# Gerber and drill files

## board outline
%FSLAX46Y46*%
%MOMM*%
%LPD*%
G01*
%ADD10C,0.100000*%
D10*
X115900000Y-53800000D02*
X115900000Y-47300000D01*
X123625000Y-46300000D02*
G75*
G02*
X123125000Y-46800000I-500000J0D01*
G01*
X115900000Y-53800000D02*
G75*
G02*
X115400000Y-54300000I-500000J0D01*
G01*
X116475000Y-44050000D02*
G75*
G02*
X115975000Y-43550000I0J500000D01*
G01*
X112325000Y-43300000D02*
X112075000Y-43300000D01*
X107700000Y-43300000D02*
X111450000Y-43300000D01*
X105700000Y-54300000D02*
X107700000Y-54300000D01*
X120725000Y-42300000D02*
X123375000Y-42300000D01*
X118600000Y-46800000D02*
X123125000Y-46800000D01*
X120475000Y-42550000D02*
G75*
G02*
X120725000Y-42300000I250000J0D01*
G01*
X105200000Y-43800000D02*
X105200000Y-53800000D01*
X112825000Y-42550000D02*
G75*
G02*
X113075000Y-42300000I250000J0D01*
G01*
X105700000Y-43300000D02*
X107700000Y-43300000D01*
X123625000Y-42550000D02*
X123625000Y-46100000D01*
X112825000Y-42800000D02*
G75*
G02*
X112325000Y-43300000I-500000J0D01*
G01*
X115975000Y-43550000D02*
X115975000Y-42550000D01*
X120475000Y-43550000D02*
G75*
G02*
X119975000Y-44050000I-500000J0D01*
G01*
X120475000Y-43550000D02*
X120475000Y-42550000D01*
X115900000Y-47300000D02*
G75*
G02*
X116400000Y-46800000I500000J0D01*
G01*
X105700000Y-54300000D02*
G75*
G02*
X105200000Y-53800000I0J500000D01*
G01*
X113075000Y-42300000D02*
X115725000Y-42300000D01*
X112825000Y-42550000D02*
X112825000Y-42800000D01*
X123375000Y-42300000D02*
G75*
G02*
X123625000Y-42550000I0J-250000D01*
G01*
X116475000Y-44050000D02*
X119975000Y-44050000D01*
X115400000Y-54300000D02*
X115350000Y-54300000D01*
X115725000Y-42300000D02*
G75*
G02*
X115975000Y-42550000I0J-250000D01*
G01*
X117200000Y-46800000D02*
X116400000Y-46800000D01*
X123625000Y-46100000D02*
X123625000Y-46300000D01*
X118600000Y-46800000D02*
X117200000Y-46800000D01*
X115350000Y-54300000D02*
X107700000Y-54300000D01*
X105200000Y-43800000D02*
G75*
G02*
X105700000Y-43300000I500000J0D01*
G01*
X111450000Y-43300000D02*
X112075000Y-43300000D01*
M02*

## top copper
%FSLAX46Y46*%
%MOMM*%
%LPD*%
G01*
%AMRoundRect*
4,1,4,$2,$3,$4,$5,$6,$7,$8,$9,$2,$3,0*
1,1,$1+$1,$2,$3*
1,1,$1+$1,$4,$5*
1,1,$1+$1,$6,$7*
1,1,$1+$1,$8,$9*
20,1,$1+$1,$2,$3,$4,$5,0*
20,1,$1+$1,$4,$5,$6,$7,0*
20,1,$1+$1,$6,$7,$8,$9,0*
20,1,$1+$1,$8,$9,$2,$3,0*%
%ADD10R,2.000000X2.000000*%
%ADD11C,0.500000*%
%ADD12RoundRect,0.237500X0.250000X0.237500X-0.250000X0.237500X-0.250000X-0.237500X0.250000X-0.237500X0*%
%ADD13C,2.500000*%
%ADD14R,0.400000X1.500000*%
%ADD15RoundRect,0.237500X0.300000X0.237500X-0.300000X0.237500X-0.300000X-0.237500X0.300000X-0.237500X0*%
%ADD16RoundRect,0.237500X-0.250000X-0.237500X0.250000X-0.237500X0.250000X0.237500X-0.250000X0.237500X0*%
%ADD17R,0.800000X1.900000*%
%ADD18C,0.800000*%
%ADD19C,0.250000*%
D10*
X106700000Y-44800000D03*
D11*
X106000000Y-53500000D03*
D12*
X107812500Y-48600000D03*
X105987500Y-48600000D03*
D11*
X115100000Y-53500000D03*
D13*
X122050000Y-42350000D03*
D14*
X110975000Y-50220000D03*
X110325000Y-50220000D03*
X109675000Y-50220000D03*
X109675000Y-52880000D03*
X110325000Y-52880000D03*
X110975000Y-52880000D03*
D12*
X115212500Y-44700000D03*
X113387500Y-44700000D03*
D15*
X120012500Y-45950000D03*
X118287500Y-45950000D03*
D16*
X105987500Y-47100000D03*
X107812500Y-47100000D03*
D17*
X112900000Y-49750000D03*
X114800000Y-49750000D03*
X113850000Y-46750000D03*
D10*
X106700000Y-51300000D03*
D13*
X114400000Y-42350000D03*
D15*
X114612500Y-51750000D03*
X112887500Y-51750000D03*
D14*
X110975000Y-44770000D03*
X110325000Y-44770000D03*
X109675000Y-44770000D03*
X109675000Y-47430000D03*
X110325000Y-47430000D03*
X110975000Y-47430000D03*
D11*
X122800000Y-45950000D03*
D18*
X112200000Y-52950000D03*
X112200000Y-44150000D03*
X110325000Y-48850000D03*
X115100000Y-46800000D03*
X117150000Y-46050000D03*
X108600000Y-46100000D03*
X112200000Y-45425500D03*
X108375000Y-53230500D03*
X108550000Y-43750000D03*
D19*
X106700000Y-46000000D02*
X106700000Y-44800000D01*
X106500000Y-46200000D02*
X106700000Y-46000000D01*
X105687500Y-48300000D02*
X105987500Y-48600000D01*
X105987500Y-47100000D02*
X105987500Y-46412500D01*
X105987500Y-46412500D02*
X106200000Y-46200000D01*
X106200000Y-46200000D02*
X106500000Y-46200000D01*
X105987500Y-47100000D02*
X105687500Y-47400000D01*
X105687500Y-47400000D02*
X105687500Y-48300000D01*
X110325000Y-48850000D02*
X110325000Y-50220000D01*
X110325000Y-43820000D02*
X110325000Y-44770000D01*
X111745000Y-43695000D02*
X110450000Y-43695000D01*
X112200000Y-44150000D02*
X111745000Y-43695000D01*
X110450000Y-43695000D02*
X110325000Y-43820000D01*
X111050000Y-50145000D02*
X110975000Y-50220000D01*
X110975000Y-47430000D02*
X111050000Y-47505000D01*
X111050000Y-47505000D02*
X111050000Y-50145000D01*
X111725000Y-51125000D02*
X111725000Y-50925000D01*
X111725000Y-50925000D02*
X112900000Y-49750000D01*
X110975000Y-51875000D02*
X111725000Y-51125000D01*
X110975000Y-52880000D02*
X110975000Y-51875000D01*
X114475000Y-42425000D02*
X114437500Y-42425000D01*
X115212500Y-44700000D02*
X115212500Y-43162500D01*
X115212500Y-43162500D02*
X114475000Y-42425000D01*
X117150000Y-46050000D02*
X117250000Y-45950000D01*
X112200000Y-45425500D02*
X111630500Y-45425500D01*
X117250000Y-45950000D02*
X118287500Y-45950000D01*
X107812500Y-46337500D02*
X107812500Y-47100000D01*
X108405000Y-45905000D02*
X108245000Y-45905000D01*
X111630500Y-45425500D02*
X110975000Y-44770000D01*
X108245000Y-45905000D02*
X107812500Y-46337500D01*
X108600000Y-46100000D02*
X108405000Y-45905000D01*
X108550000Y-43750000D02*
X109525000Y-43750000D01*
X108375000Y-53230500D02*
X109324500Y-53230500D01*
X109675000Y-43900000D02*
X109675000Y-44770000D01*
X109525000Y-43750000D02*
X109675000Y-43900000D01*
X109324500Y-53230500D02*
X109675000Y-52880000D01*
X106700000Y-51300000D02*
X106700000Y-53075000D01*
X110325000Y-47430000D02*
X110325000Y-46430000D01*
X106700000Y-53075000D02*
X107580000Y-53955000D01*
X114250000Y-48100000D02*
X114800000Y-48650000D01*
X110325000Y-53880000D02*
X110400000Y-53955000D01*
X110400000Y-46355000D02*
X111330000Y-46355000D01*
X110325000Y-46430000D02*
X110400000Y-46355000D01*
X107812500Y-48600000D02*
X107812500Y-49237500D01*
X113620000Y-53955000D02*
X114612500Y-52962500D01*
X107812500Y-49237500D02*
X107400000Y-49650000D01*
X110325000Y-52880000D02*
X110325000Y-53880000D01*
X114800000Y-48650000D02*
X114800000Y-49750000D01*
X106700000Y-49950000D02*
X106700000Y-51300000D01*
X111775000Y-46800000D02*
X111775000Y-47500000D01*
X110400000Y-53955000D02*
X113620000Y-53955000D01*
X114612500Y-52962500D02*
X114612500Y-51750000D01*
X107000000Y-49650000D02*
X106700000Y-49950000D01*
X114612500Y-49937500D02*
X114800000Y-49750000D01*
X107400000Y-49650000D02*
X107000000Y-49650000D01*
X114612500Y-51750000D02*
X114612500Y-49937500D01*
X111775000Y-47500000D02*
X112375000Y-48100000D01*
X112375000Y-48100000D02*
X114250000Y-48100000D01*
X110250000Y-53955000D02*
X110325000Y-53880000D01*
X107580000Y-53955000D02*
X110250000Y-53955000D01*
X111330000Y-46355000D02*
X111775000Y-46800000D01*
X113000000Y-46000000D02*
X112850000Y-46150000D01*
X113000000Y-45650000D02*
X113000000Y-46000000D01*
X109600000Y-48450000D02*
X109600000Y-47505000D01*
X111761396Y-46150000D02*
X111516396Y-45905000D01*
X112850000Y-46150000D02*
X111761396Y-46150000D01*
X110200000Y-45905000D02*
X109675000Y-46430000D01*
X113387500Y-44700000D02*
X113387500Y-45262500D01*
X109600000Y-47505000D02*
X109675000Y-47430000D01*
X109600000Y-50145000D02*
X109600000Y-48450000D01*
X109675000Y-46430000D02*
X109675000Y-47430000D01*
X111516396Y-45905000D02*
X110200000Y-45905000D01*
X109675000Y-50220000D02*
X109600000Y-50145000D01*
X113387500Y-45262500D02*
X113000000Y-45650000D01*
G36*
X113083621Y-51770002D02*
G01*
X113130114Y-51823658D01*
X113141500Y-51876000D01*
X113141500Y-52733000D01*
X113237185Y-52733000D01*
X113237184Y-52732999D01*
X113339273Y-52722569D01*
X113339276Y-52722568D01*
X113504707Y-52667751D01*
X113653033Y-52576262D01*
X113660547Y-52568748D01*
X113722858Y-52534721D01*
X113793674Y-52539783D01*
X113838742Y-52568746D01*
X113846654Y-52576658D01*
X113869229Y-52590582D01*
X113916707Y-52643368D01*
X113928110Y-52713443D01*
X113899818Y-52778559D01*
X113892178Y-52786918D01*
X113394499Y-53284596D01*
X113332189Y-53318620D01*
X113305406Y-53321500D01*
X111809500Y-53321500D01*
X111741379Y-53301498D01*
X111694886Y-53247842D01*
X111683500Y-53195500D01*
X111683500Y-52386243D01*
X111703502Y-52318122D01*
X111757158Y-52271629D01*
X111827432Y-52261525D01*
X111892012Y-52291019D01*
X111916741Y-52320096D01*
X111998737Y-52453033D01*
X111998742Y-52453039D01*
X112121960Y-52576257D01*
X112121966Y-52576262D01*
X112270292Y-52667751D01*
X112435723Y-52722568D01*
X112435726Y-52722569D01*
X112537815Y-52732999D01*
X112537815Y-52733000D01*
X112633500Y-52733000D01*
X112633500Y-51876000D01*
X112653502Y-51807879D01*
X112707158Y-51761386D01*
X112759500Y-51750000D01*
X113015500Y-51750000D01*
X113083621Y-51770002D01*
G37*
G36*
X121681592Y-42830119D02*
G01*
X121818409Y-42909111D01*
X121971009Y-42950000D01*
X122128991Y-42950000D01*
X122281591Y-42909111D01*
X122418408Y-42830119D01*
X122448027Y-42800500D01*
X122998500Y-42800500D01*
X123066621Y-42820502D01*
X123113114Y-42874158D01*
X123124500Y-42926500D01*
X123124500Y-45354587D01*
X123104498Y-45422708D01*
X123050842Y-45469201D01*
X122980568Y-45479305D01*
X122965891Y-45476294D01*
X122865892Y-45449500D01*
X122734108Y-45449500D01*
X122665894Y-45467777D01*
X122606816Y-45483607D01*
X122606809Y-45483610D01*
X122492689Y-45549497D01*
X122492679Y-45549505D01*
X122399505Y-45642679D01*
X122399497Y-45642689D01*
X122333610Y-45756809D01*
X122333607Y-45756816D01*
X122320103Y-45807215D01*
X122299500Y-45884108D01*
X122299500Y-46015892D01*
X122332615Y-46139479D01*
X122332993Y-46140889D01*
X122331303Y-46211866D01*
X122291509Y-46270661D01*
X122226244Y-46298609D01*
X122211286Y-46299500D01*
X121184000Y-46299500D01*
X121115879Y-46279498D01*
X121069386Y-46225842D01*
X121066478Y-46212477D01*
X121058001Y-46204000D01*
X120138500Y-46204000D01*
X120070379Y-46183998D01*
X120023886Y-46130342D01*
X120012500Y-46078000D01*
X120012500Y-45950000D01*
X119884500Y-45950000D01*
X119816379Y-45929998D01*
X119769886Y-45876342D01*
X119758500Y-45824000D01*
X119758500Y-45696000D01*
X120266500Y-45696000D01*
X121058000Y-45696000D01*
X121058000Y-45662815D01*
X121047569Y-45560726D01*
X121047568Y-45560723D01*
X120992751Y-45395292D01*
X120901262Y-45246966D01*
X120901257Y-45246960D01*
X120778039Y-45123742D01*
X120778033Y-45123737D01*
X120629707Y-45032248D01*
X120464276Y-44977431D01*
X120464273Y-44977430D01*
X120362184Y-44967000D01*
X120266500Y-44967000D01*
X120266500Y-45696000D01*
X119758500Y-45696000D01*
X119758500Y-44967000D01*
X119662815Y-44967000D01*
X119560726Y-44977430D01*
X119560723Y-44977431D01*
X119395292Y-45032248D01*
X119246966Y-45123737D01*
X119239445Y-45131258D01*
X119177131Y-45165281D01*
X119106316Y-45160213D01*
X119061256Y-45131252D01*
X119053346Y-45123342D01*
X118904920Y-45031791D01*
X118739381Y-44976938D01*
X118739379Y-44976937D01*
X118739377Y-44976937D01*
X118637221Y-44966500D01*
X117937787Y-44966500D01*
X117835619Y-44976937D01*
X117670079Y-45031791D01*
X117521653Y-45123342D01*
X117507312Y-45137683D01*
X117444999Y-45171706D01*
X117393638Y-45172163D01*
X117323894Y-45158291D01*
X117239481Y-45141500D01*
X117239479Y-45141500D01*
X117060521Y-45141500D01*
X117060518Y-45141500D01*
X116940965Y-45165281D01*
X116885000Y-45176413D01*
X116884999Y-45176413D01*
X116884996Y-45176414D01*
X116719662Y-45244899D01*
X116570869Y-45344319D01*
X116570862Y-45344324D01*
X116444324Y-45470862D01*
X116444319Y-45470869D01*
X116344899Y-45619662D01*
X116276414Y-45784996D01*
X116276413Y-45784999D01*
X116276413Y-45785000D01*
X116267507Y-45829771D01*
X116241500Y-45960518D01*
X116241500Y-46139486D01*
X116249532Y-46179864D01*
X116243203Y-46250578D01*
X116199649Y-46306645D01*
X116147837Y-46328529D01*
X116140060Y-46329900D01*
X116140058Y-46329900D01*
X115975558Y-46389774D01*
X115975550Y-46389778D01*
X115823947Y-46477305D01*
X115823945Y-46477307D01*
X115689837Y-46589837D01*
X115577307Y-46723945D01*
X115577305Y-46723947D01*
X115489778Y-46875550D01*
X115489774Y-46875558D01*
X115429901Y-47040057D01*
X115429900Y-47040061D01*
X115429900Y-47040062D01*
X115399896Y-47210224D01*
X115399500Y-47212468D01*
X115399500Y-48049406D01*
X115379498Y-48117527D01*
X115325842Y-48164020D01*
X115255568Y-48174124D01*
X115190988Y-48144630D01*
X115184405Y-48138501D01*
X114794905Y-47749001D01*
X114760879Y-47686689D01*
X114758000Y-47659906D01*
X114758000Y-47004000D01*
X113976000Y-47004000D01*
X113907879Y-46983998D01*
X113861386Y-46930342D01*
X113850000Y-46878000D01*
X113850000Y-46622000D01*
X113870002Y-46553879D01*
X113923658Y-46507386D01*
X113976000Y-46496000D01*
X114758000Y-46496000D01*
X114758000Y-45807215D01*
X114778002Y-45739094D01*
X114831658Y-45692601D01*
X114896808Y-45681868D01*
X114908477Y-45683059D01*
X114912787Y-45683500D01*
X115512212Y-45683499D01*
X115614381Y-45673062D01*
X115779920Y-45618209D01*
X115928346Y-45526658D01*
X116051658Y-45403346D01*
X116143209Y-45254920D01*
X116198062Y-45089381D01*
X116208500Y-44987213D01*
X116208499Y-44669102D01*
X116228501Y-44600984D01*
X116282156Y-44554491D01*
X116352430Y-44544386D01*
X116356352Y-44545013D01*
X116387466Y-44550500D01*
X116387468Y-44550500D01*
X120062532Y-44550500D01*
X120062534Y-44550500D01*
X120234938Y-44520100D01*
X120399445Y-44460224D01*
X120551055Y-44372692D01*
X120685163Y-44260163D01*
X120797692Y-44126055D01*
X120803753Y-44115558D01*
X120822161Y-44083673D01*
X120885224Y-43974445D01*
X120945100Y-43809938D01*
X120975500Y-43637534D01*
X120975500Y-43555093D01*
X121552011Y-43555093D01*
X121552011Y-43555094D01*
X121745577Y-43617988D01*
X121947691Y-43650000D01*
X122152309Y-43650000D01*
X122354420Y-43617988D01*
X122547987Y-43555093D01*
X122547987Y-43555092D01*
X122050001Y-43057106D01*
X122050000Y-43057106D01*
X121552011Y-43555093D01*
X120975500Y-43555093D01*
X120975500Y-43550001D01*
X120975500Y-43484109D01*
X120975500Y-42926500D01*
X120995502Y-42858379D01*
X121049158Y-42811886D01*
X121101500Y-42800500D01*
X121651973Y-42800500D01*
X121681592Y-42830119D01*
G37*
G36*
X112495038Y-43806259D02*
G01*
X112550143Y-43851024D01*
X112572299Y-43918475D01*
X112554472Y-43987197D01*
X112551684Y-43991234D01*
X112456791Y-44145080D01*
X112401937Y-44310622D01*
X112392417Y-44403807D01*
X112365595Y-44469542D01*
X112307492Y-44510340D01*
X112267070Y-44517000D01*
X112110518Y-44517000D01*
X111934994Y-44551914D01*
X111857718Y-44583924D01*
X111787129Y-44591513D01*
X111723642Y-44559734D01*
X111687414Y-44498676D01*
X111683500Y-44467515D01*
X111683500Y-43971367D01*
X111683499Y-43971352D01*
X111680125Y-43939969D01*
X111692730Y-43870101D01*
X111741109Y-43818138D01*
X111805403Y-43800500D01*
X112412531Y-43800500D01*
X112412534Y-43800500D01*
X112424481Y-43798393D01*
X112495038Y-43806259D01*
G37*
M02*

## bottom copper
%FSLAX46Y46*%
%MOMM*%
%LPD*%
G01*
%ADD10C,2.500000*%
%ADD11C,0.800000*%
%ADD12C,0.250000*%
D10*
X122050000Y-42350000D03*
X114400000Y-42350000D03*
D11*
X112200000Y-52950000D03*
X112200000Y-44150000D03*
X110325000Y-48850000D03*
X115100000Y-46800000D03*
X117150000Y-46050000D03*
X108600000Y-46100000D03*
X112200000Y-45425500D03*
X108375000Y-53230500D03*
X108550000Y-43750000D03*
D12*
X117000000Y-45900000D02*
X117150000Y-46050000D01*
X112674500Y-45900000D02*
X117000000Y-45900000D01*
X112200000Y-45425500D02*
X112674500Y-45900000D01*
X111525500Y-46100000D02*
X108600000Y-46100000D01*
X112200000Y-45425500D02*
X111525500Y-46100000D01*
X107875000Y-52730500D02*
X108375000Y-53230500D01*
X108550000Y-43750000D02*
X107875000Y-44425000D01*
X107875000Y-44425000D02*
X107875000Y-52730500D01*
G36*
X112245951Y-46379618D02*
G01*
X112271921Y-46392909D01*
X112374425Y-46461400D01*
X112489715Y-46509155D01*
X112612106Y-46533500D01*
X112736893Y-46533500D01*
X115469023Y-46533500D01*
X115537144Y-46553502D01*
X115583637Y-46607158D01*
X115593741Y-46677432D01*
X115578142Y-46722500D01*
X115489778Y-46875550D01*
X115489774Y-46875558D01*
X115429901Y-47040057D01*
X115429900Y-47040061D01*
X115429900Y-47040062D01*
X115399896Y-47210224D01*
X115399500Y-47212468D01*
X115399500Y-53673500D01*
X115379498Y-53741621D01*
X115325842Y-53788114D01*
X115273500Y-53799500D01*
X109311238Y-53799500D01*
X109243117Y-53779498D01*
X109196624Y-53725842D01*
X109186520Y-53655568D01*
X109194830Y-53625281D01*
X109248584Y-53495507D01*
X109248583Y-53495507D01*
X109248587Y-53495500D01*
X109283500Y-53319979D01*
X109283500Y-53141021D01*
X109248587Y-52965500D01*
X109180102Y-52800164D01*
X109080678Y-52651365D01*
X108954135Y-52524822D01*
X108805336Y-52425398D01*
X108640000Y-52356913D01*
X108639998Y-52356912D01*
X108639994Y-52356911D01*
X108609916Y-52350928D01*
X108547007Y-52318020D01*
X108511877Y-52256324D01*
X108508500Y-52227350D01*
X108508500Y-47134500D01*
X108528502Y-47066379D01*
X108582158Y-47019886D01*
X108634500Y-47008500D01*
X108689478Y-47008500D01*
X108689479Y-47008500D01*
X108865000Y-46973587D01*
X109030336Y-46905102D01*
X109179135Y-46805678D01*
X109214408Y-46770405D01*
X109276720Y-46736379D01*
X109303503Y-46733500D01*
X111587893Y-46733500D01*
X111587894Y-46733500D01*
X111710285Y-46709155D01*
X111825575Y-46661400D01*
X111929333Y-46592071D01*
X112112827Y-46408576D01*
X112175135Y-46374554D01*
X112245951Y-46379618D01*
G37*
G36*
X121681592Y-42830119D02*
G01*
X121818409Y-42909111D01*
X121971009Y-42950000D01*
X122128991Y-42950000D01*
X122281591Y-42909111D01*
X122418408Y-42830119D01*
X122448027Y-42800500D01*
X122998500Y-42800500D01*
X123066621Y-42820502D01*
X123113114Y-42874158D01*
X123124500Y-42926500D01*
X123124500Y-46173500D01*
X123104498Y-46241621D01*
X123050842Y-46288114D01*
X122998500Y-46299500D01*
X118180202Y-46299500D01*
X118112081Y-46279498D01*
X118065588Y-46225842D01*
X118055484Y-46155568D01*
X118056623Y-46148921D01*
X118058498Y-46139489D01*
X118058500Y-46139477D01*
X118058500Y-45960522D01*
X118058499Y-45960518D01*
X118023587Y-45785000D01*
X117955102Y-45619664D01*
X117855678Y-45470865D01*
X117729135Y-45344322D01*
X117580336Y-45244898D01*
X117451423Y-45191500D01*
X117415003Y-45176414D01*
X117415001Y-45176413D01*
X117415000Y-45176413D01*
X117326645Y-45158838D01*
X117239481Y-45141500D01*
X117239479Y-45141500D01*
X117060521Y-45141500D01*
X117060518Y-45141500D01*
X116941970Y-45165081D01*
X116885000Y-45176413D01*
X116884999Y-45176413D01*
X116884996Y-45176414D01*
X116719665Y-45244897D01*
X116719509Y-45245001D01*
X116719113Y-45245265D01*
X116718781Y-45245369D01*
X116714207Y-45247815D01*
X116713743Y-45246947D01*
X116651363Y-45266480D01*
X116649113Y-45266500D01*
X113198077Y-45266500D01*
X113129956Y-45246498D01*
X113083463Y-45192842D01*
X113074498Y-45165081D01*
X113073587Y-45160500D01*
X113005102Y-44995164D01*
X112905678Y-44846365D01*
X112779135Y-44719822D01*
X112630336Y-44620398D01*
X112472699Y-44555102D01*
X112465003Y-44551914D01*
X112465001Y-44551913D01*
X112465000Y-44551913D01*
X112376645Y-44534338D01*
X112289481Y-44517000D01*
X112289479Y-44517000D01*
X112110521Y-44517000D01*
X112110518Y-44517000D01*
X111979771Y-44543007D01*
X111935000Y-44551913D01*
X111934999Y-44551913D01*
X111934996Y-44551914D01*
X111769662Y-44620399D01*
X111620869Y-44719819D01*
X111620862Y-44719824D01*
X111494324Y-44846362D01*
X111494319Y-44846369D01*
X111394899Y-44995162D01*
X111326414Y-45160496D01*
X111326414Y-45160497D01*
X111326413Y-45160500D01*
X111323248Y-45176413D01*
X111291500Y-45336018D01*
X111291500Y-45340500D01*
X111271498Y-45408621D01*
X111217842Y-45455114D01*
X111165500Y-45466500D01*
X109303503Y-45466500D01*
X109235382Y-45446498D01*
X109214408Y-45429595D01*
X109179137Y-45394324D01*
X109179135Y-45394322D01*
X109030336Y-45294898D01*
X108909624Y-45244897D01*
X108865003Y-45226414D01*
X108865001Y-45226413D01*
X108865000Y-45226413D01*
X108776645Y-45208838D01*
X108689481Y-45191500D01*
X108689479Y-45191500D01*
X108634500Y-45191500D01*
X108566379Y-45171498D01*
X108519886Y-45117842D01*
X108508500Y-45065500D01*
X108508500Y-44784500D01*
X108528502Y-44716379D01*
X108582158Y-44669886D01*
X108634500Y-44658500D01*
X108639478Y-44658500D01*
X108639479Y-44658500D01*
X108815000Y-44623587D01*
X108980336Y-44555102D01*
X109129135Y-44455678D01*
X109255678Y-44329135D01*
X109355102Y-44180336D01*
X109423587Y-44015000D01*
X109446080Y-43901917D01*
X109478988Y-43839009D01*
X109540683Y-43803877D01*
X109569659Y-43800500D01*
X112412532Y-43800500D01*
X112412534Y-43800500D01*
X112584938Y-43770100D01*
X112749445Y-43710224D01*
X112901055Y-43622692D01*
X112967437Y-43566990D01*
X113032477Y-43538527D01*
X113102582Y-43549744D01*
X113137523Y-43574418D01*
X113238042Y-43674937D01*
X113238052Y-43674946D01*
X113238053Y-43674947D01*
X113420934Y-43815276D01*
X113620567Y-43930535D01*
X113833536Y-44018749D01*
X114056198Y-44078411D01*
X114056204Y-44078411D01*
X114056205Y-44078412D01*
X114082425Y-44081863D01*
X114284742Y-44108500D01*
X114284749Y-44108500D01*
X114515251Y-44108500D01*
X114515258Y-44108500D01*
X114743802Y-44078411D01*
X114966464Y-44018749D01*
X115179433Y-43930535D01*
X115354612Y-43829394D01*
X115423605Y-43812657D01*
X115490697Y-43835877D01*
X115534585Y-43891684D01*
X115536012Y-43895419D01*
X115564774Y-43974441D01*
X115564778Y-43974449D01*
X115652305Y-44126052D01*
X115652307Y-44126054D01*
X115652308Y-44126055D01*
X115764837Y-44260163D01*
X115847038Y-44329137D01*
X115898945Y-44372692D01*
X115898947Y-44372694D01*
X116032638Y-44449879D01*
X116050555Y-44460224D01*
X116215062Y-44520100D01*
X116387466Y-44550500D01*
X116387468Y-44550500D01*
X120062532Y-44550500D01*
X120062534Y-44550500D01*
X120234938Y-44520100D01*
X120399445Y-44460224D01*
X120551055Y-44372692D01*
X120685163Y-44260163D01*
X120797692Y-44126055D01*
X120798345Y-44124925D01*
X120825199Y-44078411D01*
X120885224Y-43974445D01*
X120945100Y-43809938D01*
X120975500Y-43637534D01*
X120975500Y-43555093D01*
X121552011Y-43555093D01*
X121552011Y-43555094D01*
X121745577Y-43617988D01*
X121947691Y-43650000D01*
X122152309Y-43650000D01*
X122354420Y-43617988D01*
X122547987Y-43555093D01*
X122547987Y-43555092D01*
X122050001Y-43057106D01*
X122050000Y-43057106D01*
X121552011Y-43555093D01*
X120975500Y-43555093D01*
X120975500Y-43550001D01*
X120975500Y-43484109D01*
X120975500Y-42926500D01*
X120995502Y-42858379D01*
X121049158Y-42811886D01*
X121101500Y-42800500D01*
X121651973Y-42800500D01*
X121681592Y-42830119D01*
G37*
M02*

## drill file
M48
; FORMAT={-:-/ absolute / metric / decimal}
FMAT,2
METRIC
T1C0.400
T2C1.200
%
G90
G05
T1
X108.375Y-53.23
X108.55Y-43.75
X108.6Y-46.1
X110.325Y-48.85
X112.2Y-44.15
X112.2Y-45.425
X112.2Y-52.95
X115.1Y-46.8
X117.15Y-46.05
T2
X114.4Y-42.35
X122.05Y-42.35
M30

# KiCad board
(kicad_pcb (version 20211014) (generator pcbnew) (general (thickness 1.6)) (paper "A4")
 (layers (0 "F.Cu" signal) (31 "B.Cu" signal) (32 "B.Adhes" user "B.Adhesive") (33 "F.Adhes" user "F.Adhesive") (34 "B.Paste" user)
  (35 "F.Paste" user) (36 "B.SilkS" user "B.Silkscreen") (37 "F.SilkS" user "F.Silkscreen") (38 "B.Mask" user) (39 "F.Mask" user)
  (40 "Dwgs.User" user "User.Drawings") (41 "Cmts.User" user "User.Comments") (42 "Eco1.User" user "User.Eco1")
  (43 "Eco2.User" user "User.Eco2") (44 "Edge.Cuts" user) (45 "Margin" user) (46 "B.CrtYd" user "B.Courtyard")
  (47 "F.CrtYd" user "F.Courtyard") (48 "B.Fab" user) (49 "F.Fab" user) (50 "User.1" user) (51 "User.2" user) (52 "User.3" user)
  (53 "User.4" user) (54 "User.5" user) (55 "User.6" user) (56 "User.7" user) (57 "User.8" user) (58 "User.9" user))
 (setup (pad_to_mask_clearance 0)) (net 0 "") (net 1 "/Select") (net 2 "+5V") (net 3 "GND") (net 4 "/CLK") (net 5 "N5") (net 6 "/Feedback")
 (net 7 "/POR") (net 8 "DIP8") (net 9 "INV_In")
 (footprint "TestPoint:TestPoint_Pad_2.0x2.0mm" (layer "F.Cu") (at 106.7 44.8 90)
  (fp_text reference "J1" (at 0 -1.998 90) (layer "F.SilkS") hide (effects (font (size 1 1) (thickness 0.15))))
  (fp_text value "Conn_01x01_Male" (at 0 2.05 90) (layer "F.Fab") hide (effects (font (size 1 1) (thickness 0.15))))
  (pad "1" smd rect (at 0 0 90) (size 2 2) (layers "F.Cu" "F.Mask") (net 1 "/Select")))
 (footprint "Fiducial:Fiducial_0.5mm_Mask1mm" (layer "F.Cu") (at 106 53.5)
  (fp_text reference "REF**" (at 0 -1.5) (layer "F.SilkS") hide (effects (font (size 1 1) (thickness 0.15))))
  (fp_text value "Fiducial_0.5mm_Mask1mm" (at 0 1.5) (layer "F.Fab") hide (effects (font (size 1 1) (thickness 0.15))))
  (pad "" smd circle (at 0 0) (size 0.5 0.5) (layers "F.Cu" "F.Mask") (solder_mask_margin 0.25) (clearance 0.25)))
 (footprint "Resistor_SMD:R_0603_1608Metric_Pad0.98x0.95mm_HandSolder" (layer "F.Cu") (at 106.9 48.6 180)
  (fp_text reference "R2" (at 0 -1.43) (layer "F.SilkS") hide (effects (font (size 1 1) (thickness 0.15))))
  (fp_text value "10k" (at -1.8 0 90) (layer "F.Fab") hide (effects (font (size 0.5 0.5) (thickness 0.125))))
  (pad "1" smd roundrect (at -0.9125 0 180) (size 0.975 0.95) (layers "F.Cu" "F.Paste" "F.Mask") (roundrect_rratio 0.25) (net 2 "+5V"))
  (pad "2" smd roundrect (at 0.9125 0 180) (size 0.975 0.95) (layers "F.Cu" "F.Paste" "F.Mask") (roundrect_rratio 0.25) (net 1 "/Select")))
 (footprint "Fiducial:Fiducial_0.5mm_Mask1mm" (layer "F.Cu") (at 115.1 53.5)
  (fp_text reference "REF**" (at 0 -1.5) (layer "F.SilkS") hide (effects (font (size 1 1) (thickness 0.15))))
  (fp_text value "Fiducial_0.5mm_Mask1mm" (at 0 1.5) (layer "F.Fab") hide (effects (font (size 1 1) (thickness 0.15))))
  (pad "" smd circle (at 0 0) (size 0.5 0.5) (layers "F.Cu" "F.Mask") (solder_mask_margin 0.25) (clearance 0.25)))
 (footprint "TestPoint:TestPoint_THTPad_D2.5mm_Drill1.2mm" (layer "F.Cu") (at 122.05 42.35)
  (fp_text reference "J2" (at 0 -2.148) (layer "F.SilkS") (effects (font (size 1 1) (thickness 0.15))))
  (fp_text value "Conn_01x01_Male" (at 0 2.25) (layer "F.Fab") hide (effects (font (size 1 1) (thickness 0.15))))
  (pad "1" thru_hole circle (at 0 0) (size 2.5 2.5) (drill 1.2) (layers *.Cu *.Mask) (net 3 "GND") (zone_connect 1) (thermal_width 1)
   (thermal_gap 0.05)))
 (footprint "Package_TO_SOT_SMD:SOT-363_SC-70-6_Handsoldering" (layer "F.Cu") (at 110.325 51.55 -90)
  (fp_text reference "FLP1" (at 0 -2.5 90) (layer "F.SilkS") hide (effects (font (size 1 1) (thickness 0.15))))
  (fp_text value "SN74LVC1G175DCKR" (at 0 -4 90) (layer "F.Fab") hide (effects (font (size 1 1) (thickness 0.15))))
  (pad "1" smd rect (at -1.33 -0.65 270) (size 1.5 0.4) (layers "F.Cu" "F.Paste" "F.Mask") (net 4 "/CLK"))
  (pad "2" smd rect (at -1.33 0 270) (size 1.5 0.4) (layers "F.Cu" "F.Paste" "F.Mask") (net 3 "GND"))
  (pad "3" smd rect (at -1.33 0.65 270) (size 1.5 0.4) (layers "F.Cu" "F.Paste" "F.Mask") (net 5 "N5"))
  (pad "4" smd rect (at 1.33 0.65 270) (size 1.5 0.4) (layers "F.Cu" "F.Paste" "F.Mask") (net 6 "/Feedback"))
  (pad "5" smd rect (at 1.33 0 270) (size 1.5 0.4) (layers "F.Cu" "F.Paste" "F.Mask") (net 2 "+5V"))
  (pad "6" smd rect (at 1.33 -0.65 270) (size 1.5 0.4) (layers "F.Cu" "F.Paste" "F.Mask") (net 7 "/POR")))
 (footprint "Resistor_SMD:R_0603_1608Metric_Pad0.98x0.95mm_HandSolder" (layer "F.Cu") (at 114.3 44.7 180)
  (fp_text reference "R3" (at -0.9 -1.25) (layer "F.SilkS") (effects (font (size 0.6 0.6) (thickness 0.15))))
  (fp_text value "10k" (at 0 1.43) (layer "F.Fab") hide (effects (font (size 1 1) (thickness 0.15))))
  (pad "1" smd roundrect (at -0.9125 0 180) (size 0.975 0.95) (layers "F.Cu" "F.Paste" "F.Mask") (roundrect_rratio 0.25) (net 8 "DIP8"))
  (pad "2" smd roundrect (at 0.9125 0 180) (size 0.975 0.95) (layers "F.Cu" "F.Paste" "F.Mask") (roundrect_rratio 0.25) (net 5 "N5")))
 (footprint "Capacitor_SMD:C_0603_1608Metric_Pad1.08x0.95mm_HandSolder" (layer "F.Cu") (at 119.15 45.95 180)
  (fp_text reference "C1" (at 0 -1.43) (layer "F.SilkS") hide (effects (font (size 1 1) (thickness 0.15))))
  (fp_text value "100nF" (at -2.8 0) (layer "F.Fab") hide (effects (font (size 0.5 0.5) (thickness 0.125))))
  (pad "1" smd roundrect (at -0.8625 0 180) (size 1.075 0.95) (layers "F.Cu" "F.Paste" "F.Mask") (roundrect_rratio 0.25) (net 3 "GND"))
  (pad "2" smd roundrect (at 0.8625 0 180) (size 1.075 0.95) (layers "F.Cu" "F.Paste" "F.Mask") (roundrect_rratio 0.25) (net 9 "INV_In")))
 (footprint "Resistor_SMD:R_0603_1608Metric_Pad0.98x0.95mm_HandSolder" (layer "F.Cu") (at 106.9 47.1)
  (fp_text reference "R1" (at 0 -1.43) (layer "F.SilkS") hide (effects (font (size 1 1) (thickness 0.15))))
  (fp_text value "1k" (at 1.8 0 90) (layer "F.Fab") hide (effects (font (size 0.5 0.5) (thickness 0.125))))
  (pad "1" smd roundrect (at -0.9125 0) (size 0.975 0.95) (layers "F.Cu" "F.Paste" "F.Mask") (roundrect_rratio 0.25) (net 1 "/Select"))
  (pad "2" smd roundrect (at 0.9125 0) (size 0.975 0.95) (layers "F.Cu" "F.Paste" "F.Mask") (roundrect_rratio 0.25) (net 9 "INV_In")))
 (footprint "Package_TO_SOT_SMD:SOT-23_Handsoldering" (layer "F.Cu") (at 113.85 48.25 90)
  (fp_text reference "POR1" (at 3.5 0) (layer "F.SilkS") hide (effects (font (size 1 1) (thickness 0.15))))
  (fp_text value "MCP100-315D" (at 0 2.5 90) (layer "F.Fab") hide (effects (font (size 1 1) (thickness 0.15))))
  (pad "1" smd rect (at -1.5 -0.95 90) (size 1.9 0.8) (layers "F.Cu" "F.Paste" "F.Mask") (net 7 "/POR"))
  (pad "2" smd rect (at -1.5 0.95 90) (size 1.9 0.8) (layers "F.Cu" "F.Paste" "F.Mask") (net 2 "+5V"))
  (pad "3" smd rect (at 1.5 0 90) (size 1.9 0.8) (layers "F.Cu" "F.Paste" "F.Mask") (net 3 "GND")))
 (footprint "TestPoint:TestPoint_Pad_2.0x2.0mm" (layer "F.Cu") (at 106.7 51.3 90)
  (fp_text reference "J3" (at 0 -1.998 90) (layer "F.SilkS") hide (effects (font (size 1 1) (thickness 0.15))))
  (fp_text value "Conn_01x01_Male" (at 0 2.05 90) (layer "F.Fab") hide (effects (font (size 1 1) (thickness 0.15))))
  (pad "1" smd rect (at 0 0 90) (size 2 2) (layers "F.Cu" "F.Mask") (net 2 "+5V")))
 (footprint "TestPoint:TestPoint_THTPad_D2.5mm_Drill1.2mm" (layer "F.Cu") (at 114.4 42.35)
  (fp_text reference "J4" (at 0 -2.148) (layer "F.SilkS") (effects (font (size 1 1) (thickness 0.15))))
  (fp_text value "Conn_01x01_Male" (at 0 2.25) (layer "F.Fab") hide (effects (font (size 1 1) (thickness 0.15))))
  (pad "1" thru_hole circle (at 0 0) (size 2.5 2.5) (drill 1.2) (layers *.Cu *.Mask) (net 8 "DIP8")))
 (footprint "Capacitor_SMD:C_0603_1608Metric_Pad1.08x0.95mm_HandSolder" (layer "F.Cu") (at 113.75 51.75 180)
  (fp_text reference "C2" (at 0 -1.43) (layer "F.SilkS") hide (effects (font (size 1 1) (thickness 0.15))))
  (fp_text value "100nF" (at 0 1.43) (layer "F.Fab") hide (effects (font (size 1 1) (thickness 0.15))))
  (pad "1" smd roundrect (at -0.8625 0 180) (size 1.075 0.95) (layers "F.Cu" "F.Paste" "F.Mask") (roundrect_rratio 0.25) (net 2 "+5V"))
  (pad "2" smd roundrect (at 0.8625 0 180) (size 1.075 0.95) (layers "F.Cu" "F.Paste" "F.Mask") (roundrect_rratio 0.25) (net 3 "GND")))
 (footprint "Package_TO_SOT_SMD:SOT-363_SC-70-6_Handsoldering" (layer "F.Cu") (at 110.325 46.1 -90)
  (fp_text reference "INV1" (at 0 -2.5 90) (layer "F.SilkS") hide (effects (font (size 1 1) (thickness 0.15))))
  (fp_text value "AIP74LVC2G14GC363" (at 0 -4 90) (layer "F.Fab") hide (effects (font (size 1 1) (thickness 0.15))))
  (pad "1" smd rect (at -1.33 -0.65 270) (size 1.5 0.4) (layers "F.Cu" "F.Paste" "F.Mask") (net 9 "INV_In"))
  (pad "2" smd rect (at -1.33 0 270) (size 1.5 0.4) (layers "F.Cu" "F.Paste" "F.Mask") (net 3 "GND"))
  (pad "3" smd rect (at -1.33 0.65 270) (size 1.5 0.4) (layers "F.Cu" "F.Paste" "F.Mask") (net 6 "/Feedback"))
  (pad "4" smd rect (at 1.33 0.65 270) (size 1.5 0.4) (layers "F.Cu" "F.Paste" "F.Mask") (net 5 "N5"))
  (pad "5" smd rect (at 1.33 0 270) (size 1.5 0.4) (layers "F.Cu" "F.Paste" "F.Mask") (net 2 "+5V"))
  (pad "6" smd rect (at 1.33 -0.65 270) (size 1.5 0.4) (layers "F.Cu" "F.Paste" "F.Mask") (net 4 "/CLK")))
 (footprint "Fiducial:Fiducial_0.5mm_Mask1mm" (layer "F.Cu") (at 122.8 45.95)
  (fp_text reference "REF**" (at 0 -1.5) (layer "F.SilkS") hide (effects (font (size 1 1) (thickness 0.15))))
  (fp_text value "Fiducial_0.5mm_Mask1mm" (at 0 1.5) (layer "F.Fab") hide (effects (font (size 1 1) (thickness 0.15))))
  (pad "" smd circle (at 0 0) (size 0.5 0.5) (layers "F.Cu" "F.Mask") (solder_mask_margin 0.25) (clearance 0.25)))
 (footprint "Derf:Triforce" (layer "B.Cu") (at 110.65 46.2 180)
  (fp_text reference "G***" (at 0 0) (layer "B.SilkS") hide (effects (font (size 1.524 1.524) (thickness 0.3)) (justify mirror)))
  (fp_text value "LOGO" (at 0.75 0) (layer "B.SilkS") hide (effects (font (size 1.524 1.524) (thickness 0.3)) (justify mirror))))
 (gr_line (start 115.9 53.8) (end 115.9 47.3) (layer "Edge.Cuts") (width 0.1))
 (gr_arc (start 123.625 46.3) (mid 123.478553 46.653553) (end 123.125 46.8) (layer "Edge.Cuts") (width 0.1))
 (gr_arc (start 115.9 53.8) (mid 115.753553 54.153553) (end 115.4 54.3) (layer "Edge.Cuts") (width 0.1))
 (gr_arc (start 116.475 44.05) (mid 116.121447 43.903553) (end 115.975 43.55) (layer "Edge.Cuts") (width 0.1))
 (gr_line (start 112.325 43.3) (end 112.075 43.3) (layer "Edge.Cuts") (width 0.1))
 (gr_line (start 107.7 43.3) (end 111.45 43.3) (layer "Edge.Cuts") (width 0.1))
 (gr_line (start 105.7 54.3) (end 107.7 54.3) (layer "Edge.Cuts") (width 0.1))
 (gr_line (start 120.725 42.3) (end 123.375 42.3) (layer "Edge.Cuts") (width 0.1))
 (gr_line (start 118.6 46.8) (end 123.125 46.8) (layer "Edge.Cuts") (width 0.1))
 (gr_arc (start 120.475 42.55) (mid 120.548223 42.373223) (end 120.725 42.3) (layer "Edge.Cuts") (width 0.1))
 (gr_line (start 105.2 43.8) (end 105.2 53.8) (layer "Edge.Cuts") (width 0.1))
 (gr_arc (start 112.825 42.55) (mid 112.898223 42.373223) (end 113.075 42.3) (layer "Edge.Cuts") (width 0.1))
 (gr_line (start 105.7 43.3) (end 107.7 43.3) (layer "Edge.Cuts") (width 0.1))
 (gr_line (start 123.625 42.55) (end 123.625 46.1) (layer "Edge.Cuts") (width 0.1))
 (gr_arc (start 112.825 42.8) (mid 112.678553 43.153553) (end 112.325 43.3) (layer "Edge.Cuts") (width 0.1))
 (gr_line (start 115.975 43.55) (end 115.975 42.55) (layer "Edge.Cuts") (width 0.1))
 (gr_arc (start 120.475 43.55) (mid 120.328553 43.903553) (end 119.975 44.05) (layer "Edge.Cuts") (width 0.1))
 (gr_line (start 120.475 43.55) (end 120.475 42.55) (layer "Edge.Cuts") (width 0.1))
 (gr_arc (start 115.9 47.3) (mid 116.046447 46.946447) (end 116.4 46.8) (layer "Edge.Cuts") (width 0.1))
 (gr_arc (start 105.7 54.3) (mid 105.346447 54.153553) (end 105.2 53.8) (layer "Edge.Cuts") (width 0.1))
 (gr_line (start 113.075 42.3) (end 115.725 42.3) (layer "Edge.Cuts") (width 0.1))
 (gr_line (start 112.825 42.55) (end 112.825 42.8) (layer "Edge.Cuts") (width 0.1))
 (gr_arc (start 123.375 42.3) (mid 123.551777 42.373223) (end 123.625 42.55) (layer "Edge.Cuts") (width 0.1))
 (gr_line (start 116.475 44.05) (end 119.975 44.05) (layer "Edge.Cuts") (width 0.1))
 (gr_line (start 115.4 54.3) (end 115.35 54.3) (layer "Edge.Cuts") (width 0.1))
 (gr_arc (start 115.725 42.3) (mid 115.901777 42.373223) (end 115.975 42.55) (layer "Edge.Cuts") (width 0.1))
 (gr_line (start 117.2 46.8) (end 116.4 46.8) (layer "Edge.Cuts") (width 0.1))
 (gr_line (start 123.625 46.1) (end 123.625 46.3) (layer "Edge.Cuts") (width 0.1))
 (gr_line (start 118.6 46.8) (end 117.2 46.8) (layer "Edge.Cuts") (width 0.1))
 (gr_line (start 115.35 54.3) (end 107.7 54.3) (layer "Edge.Cuts") (width 0.1))
 (gr_arc (start 105.2 43.8) (mid 105.346447 43.446447) (end 105.7 43.3) (layer "Edge.Cuts") (width 0.1))
 (gr_line (start 111.45 43.3) (end 112.075 43.3) (layer "Edge.Cuts") (width 0.1))
 (segment (start 106.7 46) (end 106.7 44.8) (width 0.25) (layer "F.Cu") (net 1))
 (segment (start 106.5 46.2) (end 106.7 46) (width 0.25) (layer "F.Cu") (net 1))
 (segment (start 105.6875 48.3) (end 105.9875 48.6) (width 0.25) (layer "F.Cu") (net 1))
 (segment (start 105.9875 47.1) (end 105.9875 46.4125) (width 0.25) (layer "F.Cu") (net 1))
 (segment (start 105.9875 46.4125) (end 106.2 46.2) (width 0.25) (layer "F.Cu") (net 1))
 (segment (start 106.2 46.2) (end 106.5 46.2) (width 0.25) (layer "F.Cu") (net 1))
 (segment (start 105.9875 47.1) (end 105.6875 47.4) (width 0.25) (layer "F.Cu") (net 1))
 (segment (start 105.6875 47.4) (end 105.6875 48.3) (width 0.25) (layer "F.Cu") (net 1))
 (segment (start 110.325 48.85) (end 110.325 50.22) (width 0.25) (layer "F.Cu") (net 3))
 (segment (start 110.325 43.82) (end 110.325 44.77) (width 0.25) (layer "F.Cu") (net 3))
 (segment (start 111.745 43.695) (end 110.45 43.695) (width 0.25) (layer "F.Cu") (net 3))
 (segment (start 112.2 44.15) (end 111.745 43.695) (width 0.25) (layer "F.Cu") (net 3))
 (segment (start 110.45 43.695) (end 110.325 43.82) (width 0.25) (layer "F.Cu") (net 3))
 (via (at 112.2 52.95) (size 0.8) (drill 0.4) (layers "F.Cu" "B.Cu") (free) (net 3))
 (via (at 112.2 44.15) (size 0.8) (drill 0.4) (layers "F.Cu" "B.Cu") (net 3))
 (via (at 110.325 48.85) (size 0.8) (drill 0.4) (layers "F.Cu" "B.Cu") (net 3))
 (via (at 115.1 46.8) (size 0.8) (drill 0.4) (layers "F.Cu" "B.Cu") (free) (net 3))
 (segment (start 111.05 50.145) (end 110.975 50.22) (width 0.25) (layer "F.Cu") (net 4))
 (segment (start 110.975 47.43) (end 111.05 47.505) (width 0.25) (layer "F.Cu") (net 4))
 (segment (start 111.05 47.505) (end 111.05 50.145) (width 0.25) (layer "F.Cu") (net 4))
 (segment (start 111.725 51.125) (end 111.725 50.925) (width 0.25) (layer "F.Cu") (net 7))
 (segment (start 111.725 50.925) (end 112.9 49.75) (width 0.25) (layer "F.Cu") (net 7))
 (segment (start 110.975 51.875) (end 111.725 51.125) (width 0.25) (layer "F.Cu") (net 7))
 (segment (start 110.975 52.88) (end 110.975 51.875) (width 0.25) (layer "F.Cu") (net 7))
 (segment (start 114.475 42.425) (end 114.4375 42.425) (width 0.25) (layer "F.Cu") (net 8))
 (segment (start 115.2125 44.7) (end 115.2125 43.1625) (width 0.25) (layer "F.Cu") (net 8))
 (segment (start 115.2125 43.1625) (end 114.475 42.425) (width 0.25) (layer "F.Cu") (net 8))
 (segment (start 117.15 46.05) (end 117.25 45.95) (width 0.25) (layer "F.Cu") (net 9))
 (segment (start 112.2 45.4255) (end 111.6305 45.4255) (width 0.25) (layer "F.Cu") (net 9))
 (segment (start 117.25 45.95) (end 118.2875 45.95) (width 0.25) (layer "F.Cu") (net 9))
 (segment (start 107.8125 46.3375) (end 107.8125 47.1) (width 0.25) (layer "F.Cu") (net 9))
 (segment (start 108.405 45.905) (end 108.245 45.905) (width 0.25) (layer "F.Cu") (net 9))
 (segment (start 111.6305 45.4255) (end 110.975 44.77) (width 0.25) (layer "F.Cu") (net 9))
 (segment (start 108.245 45.905) (end 107.8125 46.3375) (width 0.25) (layer "F.Cu") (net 9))
 (segment (start 108.6 46.1) (end 108.405 45.905) (width 0.25) (layer "F.Cu") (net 9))
 (via (at 117.15 46.05) (size 0.8) (drill 0.4) (layers "F.Cu" "B.Cu") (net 9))
 (via (at 108.6 46.1) (size 0.8) (drill 0.4) (layers "F.Cu" "B.Cu") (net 9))
 (via (at 112.2 45.4255) (size 0.8) (drill 0.4) (layers "F.Cu" "B.Cu") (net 9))
 (segment (start 117 45.9) (end 117.15 46.05) (width 0.25) (layer "B.Cu") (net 9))
 (segment (start 112.6745 45.9) (end 117 45.9) (width 0.25) (layer "B.Cu") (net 9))
 (segment (start 112.2 45.4255) (end 112.6745 45.9) (width 0.25) (layer "B.Cu") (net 9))
 (segment (start 111.5255 46.1) (end 108.6 46.1) (width 0.25) (layer "B.Cu") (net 9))
 (segment (start 112.2 45.4255) (end 111.5255 46.1) (width 0.25) (layer "B.Cu") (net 9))
 (segment (start 108.55 43.75) (end 109.525 43.75) (width 0.25) (layer "F.Cu") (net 6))
 (segment (start 108.375 53.2305) (end 109.3245 53.2305) (width 0.25) (layer "F.Cu") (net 6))
 (segment (start 109.675 43.9) (end 109.675 44.77) (width 0.25) (layer "F.Cu") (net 6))
 (segment (start 109.525 43.75) (end 109.675 43.9) (width 0.25) (layer "F.Cu") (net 6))
 (segment (start 109.3245 53.2305) (end 109.675 52.88) (width 0.25) (layer "F.Cu") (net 6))
 (via (at 108.375 53.2305) (size 0.8) (drill 0.4) (layers "F.Cu" "B.Cu") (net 6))
 (via (at 108.55 43.75) (size 0.8) (drill 0.4) (layers "F.Cu" "B.Cu") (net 6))
 (segment (start 107.875 52.7305) (end 108.375 53.2305) (width 0.25) (layer "B.Cu") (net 6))
 (segment (start 108.55 43.75) (end 107.875 44.425) (width 0.25) (layer "B.Cu") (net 6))
 (segment (start 107.875 44.425) (end 107.875 52.7305) (width 0.25) (layer "B.Cu") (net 6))
 (segment (start 106.7 51.3) (end 106.7 53.075) (width 0.25) (layer "F.Cu") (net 2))
 (segment (start 110.325 47.43) (end 110.325 46.43) (width 0.25) (layer "F.Cu") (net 2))
 (segment (start 106.7 53.075) (end 107.58 53.955) (width 0.25) (layer "F.Cu") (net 2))
 (segment (start 114.25 48.1) (end 114.8 48.65) (width 0.25) (layer "F.Cu") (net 2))
 (segment (start 110.325 53.88) (end 110.4 53.955) (width 0.25) (layer "F.Cu") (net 2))
 (segment (start 110.4 46.355) (end 111.33 46.355) (width 0.25) (layer "F.Cu") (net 2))
 (segment (start 110.325 46.43) (end 110.4 46.355) (width 0.25) (layer "F.Cu") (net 2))
 (segment (start 107.8125 48.6) (end 107.8125 49.2375) (width 0.25) (layer "F.Cu") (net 2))
 (segment (start 113.62 53.955) (end 114.6125 52.9625) (width 0.25) (layer "F.Cu") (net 2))
 (segment (start 107.8125 49.2375) (end 107.4 49.65) (width 0.25) (layer "F.Cu") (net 2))
 (segment (start 110.325 52.88) (end 110.325 53.88) (width 0.25) (layer "F.Cu") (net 2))
 (segment (start 114.8 48.65) (end 114.8 49.75) (width 0.25) (layer "F.Cu") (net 2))
 (segment (start 106.7 49.95) (end 106.7 51.3) (width 0.25) (layer "F.Cu") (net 2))
 (segment (start 111.775 46.8) (end 111.775 47.5) (width 0.25) (layer "F.Cu") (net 2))
 (segment (start 110.4 53.955) (end 113.62 53.955) (width 0.25) (layer "F.Cu") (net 2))
 (segment (start 114.6125 52.9625) (end 114.6125 51.75) (width 0.25) (layer "F.Cu") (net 2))
 (segment (start 107 49.65) (end 106.7 49.95) (width 0.25) (layer "F.Cu") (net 2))
 (segment (start 114.6125 49.9375) (end 114.8 49.75) (width 0.25) (layer "F.Cu") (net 2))
 (segment (start 107.4 49.65) (end 107 49.65) (width 0.25) (layer "F.Cu") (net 2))
 (segment (start 114.6125 51.75) (end 114.6125 49.9375) (width 0.25) (layer "F.Cu") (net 2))
 (segment (start 111.775 47.5) (end 112.375 48.1) (width 0.25) (layer "F.Cu") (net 2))
 (segment (start 112.375 48.1) (end 114.25 48.1) (width 0.25) (layer "F.Cu") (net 2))
 (segment (start 110.25 53.955) (end 110.325 53.88) (width 0.25) (layer "F.Cu") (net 2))
 (segment (start 107.58 53.955) (end 110.25 53.955) (width 0.25) (layer "F.Cu") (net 2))
 (segment (start 111.33 46.355) (end 111.775 46.8) (width 0.25) (layer "F.Cu") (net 2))
 (segment (start 113 46) (end 112.85 46.15) (width 0.25) (layer "F.Cu") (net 5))
 (segment (start 113 45.65) (end 113 46) (width 0.25) (layer "F.Cu") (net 5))
 (segment (start 109.6 48.45) (end 109.6 47.505) (width 0.25) (layer "F.Cu") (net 5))
 (segment (start 111.761396 46.15) (end 111.516396 45.905) (width 0.25) (layer "F.Cu") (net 5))
 (segment (start 112.85 46.15) (end 111.761396 46.15) (width 0.25) (layer "F.Cu") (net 5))
 (segment (start 110.2 45.905) (end 109.675 46.43) (width 0.25) (layer "F.Cu") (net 5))
 (segment (start 113.3875 44.7) (end 113.3875 45.2625) (width 0.25) (layer "F.Cu") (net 5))
 (segment (start 109.6 47.505) (end 109.675 47.43) (width 0.25) (layer "F.Cu") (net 5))
 (segment (start 109.6 50.145) (end 109.6 48.45) (width 0.25) (layer "F.Cu") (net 5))
 (segment (start 109.675 46.43) (end 109.675 47.43) (width 0.25) (layer "F.Cu") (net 5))
 (segment (start 111.516396 45.905) (end 110.2 45.905) (width 0.25) (layer "F.Cu") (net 5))
 (segment (start 109.675 50.22) (end 109.6 50.145) (width 0.25) (layer "F.Cu") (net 5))
 (segment (start 113.3875 45.2625) (end 113 45.65) (width 0.25) (layer "F.Cu") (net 5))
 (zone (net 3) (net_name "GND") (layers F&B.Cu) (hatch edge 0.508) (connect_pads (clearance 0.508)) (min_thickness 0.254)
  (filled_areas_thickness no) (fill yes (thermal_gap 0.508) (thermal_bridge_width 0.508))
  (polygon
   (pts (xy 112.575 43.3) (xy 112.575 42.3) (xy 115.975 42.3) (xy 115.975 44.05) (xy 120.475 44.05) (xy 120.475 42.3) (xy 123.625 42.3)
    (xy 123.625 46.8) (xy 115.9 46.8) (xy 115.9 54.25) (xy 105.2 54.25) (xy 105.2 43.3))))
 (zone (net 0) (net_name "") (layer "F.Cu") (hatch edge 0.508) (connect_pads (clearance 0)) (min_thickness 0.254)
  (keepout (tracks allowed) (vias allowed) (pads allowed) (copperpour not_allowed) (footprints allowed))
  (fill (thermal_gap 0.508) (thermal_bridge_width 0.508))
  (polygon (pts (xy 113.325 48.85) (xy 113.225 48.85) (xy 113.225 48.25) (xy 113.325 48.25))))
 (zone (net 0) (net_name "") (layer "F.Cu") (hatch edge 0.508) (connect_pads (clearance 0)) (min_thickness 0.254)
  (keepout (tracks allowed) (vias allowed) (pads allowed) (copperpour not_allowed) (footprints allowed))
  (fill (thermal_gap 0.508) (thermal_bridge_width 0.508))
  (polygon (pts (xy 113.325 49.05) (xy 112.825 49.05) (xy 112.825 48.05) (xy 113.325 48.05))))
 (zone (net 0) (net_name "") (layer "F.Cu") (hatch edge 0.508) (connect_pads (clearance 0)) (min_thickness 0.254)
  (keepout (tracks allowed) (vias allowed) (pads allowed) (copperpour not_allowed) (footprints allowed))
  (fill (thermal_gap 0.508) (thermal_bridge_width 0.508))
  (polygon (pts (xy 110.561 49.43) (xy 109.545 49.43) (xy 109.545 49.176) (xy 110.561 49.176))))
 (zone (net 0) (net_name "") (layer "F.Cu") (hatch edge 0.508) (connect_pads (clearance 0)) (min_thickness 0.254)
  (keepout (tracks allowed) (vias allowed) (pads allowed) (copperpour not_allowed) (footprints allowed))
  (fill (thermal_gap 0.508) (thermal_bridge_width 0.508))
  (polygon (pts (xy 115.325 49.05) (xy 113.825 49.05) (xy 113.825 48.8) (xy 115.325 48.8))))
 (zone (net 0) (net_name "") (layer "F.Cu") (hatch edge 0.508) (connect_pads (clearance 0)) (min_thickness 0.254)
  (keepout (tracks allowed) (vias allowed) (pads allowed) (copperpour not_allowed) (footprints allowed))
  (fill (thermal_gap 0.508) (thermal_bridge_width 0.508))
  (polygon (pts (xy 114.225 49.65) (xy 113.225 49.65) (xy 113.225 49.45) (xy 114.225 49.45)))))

